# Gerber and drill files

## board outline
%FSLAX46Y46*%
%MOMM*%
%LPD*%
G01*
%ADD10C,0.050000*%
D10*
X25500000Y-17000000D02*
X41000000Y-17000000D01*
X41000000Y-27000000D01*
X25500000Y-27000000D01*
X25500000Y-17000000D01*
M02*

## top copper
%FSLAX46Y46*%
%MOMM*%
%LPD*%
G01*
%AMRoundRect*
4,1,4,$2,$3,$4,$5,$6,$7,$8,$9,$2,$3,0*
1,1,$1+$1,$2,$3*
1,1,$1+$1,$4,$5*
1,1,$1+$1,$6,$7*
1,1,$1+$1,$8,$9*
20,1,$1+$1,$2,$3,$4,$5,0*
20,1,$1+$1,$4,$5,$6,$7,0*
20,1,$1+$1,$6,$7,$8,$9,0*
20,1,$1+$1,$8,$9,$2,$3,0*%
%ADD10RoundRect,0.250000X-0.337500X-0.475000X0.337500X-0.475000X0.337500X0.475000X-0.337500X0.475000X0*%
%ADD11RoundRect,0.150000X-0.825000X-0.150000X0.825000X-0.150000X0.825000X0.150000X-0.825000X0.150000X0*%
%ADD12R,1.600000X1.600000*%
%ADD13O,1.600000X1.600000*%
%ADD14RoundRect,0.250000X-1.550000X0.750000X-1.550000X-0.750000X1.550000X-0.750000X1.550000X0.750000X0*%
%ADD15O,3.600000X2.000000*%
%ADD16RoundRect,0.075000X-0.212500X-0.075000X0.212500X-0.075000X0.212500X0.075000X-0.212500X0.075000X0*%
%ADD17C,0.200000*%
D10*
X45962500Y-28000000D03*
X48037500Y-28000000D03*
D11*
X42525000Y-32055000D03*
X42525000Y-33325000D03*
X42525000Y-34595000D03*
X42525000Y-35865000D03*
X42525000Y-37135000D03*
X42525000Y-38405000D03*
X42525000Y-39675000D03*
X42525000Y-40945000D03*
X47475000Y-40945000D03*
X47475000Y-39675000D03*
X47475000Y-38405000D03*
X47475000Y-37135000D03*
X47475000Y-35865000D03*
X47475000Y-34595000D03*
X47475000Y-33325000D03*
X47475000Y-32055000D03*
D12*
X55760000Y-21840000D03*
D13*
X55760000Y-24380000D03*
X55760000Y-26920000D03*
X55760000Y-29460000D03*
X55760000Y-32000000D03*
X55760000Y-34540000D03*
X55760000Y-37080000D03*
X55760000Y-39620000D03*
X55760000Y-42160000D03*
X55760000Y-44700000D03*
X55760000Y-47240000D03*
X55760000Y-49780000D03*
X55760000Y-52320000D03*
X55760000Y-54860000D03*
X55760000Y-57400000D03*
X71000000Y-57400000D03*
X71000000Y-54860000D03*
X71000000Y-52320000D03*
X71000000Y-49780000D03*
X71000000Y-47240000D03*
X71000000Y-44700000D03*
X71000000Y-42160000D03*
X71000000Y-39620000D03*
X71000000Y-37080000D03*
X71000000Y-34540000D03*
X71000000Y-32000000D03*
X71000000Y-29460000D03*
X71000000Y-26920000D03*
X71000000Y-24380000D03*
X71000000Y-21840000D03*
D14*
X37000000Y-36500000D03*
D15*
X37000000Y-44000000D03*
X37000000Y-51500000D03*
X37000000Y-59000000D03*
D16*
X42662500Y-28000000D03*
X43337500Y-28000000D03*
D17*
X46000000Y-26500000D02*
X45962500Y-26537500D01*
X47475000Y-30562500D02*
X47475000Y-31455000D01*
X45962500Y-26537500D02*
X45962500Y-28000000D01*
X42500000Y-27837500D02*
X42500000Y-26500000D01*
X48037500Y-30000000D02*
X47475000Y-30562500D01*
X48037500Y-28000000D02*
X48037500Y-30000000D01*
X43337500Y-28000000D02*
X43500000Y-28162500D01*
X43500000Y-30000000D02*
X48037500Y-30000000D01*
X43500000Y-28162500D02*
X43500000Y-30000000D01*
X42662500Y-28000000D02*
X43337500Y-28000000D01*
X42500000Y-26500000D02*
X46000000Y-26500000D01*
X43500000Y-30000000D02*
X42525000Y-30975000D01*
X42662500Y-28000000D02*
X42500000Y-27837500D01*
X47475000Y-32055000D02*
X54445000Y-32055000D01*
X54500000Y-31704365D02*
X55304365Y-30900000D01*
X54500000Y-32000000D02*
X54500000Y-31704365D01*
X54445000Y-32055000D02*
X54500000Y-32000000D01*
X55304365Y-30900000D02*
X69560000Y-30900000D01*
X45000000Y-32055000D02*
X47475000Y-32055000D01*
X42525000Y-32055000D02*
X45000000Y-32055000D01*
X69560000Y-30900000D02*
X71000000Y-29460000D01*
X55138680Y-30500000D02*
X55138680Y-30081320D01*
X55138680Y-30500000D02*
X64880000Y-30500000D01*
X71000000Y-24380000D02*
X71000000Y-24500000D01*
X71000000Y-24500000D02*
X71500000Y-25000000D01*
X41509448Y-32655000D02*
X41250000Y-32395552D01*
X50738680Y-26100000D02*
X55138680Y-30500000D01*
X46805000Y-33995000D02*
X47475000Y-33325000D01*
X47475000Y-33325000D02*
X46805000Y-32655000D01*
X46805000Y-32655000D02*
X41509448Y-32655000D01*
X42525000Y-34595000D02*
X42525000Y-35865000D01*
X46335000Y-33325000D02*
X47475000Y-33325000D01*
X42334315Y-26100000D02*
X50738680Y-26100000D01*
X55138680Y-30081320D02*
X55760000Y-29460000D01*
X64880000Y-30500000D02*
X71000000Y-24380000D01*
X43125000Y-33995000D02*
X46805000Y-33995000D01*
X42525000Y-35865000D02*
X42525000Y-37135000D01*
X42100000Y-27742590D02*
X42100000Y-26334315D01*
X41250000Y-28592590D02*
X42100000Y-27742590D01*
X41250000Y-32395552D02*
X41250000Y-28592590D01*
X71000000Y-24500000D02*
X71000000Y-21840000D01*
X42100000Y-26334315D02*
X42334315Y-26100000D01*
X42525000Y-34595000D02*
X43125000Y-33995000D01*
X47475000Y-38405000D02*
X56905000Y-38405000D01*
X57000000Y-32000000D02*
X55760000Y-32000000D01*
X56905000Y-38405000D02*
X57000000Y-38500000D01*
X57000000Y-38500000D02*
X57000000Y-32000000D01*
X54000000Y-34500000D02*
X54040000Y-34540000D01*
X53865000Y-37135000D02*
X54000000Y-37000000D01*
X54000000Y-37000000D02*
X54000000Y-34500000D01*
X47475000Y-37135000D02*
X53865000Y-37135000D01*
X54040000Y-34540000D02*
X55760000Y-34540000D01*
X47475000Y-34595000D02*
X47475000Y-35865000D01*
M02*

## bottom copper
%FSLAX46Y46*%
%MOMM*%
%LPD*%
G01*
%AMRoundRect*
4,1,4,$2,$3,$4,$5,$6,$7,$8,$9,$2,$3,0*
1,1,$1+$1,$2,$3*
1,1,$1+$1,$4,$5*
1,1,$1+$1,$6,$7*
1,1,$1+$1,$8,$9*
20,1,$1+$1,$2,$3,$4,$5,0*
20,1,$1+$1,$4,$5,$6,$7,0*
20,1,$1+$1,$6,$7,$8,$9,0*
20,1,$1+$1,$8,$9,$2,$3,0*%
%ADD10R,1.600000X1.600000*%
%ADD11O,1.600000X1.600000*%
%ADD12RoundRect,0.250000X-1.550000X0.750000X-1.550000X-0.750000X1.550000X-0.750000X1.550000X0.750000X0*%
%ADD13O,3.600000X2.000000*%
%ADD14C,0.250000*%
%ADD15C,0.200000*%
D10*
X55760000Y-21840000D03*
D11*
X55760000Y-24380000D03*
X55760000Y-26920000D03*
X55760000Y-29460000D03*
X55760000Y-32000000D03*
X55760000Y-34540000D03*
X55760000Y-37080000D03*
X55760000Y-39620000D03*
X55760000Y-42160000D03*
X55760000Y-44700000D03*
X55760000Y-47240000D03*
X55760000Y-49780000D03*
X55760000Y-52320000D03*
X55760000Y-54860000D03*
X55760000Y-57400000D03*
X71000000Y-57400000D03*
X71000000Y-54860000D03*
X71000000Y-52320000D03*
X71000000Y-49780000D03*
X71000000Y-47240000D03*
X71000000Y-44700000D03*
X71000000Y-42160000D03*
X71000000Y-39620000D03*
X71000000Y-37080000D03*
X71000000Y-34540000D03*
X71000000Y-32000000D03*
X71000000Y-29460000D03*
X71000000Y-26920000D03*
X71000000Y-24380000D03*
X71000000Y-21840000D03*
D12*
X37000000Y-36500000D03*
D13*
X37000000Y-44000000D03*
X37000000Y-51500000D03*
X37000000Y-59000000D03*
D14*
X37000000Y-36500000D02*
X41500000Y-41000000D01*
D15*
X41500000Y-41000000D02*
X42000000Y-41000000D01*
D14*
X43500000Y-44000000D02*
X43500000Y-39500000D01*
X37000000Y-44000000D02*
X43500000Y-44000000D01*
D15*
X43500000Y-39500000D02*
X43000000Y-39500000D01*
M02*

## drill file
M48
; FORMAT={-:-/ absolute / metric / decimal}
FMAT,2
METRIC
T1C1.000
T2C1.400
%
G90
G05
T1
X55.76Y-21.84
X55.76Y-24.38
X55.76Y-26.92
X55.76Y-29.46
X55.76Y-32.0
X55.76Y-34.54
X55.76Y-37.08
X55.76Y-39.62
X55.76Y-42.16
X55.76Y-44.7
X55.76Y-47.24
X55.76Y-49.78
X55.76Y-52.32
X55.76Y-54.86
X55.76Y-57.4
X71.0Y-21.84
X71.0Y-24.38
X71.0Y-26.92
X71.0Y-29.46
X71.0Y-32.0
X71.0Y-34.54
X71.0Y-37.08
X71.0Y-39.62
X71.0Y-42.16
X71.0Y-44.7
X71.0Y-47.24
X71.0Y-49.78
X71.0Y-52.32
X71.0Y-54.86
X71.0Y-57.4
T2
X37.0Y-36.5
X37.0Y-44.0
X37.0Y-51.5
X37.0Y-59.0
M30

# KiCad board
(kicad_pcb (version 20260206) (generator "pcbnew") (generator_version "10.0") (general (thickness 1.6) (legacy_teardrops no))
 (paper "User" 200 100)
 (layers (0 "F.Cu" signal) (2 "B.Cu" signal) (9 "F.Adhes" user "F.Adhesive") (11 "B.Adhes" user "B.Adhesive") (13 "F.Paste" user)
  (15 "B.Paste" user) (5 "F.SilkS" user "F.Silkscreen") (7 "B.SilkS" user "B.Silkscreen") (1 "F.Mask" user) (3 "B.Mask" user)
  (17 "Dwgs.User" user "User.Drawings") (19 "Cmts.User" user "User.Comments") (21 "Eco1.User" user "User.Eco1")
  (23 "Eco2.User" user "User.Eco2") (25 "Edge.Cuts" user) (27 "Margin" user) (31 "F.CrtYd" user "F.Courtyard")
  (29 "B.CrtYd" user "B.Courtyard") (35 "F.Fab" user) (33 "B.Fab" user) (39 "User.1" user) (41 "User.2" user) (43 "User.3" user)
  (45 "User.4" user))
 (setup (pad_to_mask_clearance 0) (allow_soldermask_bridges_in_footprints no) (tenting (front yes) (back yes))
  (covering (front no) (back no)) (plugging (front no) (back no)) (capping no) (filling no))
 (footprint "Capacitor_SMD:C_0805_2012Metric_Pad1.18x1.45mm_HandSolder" (layer "F.Cu") (at 47 28)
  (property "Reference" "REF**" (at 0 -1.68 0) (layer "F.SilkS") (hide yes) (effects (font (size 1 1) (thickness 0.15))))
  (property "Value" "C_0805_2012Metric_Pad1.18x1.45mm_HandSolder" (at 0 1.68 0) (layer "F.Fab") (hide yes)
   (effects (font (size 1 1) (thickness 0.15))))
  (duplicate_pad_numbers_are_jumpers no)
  (pad "1" smd roundrect (at -1.0375 0) (size 1.175 1.45) (layers "F.Cu" "F.Mask" "F.Paste") (roundrect_rratio 0.212766))
  (pad "2" smd roundrect (at 1.0375 0) (size 1.175 1.45) (layers "F.Cu" "F.Mask" "F.Paste") (roundrect_rratio 0.212766)))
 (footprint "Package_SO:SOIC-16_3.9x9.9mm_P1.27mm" (layer "F.Cu") (at 45 36.5)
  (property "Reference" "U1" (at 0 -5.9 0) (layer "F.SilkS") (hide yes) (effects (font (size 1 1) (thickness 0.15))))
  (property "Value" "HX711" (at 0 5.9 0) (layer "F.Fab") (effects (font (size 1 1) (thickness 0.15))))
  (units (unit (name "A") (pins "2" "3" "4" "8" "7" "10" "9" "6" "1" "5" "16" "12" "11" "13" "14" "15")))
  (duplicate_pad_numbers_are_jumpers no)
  (pad "1" smd roundrect (at -2.475 -4.445) (size 1.95 0.6) (layers "F.Cu" "F.Mask" "F.Paste") (roundrect_rratio 0.25)
   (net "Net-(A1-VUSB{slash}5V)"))
  (pad "2" smd roundrect (at -2.475 -3.175) (size 1.95 0.6) (layers "F.Cu" "F.Mask" "F.Paste") (roundrect_rratio 0.25)
   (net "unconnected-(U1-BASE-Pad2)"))
  (pad "3" smd roundrect (at -2.475 -1.905) (size 1.95 0.6) (layers "F.Cu" "F.Mask" "F.Paste") (roundrect_rratio 0.25) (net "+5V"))
  (pad "4" smd roundrect (at -2.475 -0.635) (size 1.95 0.6) (layers "F.Cu" "F.Mask" "F.Paste") (roundrect_rratio 0.25) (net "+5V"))
  (pad "5" smd roundrect (at -2.475 0.635) (size 1.95 0.6) (layers "F.Cu" "F.Mask" "F.Paste") (roundrect_rratio 0.25) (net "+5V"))
  (pad "6" smd roundrect (at -2.475 1.905) (size 1.95 0.6) (layers "F.Cu" "F.Mask" "F.Paste") (roundrect_rratio 0.25)
   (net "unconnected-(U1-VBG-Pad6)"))
  (pad "7" smd roundrect (at -2.475 3.175) (size 1.95 0.6) (layers "F.Cu" "F.Mask" "F.Paste") (roundrect_rratio 0.25) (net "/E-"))
  (pad "8" smd roundrect (at -2.475 4.445) (size 1.95 0.6) (layers "F.Cu" "F.Mask" "F.Paste") (roundrect_rratio 0.25) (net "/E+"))
  (pad "9" smd roundrect (at 2.475 4.445) (size 1.95 0.6) (layers "F.Cu" "F.Mask" "F.Paste") (roundrect_rratio 0.25)
   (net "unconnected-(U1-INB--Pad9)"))
  (pad "10" smd roundrect (at 2.475 3.175) (size 1.95 0.6) (layers "F.Cu" "F.Mask" "F.Paste") (roundrect_rratio 0.25)
   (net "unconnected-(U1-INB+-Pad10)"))
  (pad "11" smd roundrect (at 2.475 1.905) (size 1.95 0.6) (layers "F.Cu" "F.Mask" "F.Paste") (roundrect_rratio 0.25) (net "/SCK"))
  (pad "12" smd roundrect (at 2.475 0.635) (size 1.95 0.6) (layers "F.Cu" "F.Mask" "F.Paste") (roundrect_rratio 0.25) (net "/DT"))
  (pad "13" smd roundrect (at 2.475 -0.635) (size 1.95 0.6) (layers "F.Cu" "F.Mask" "F.Paste") (roundrect_rratio 0.25) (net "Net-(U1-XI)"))
  (pad "14" smd roundrect (at 2.475 -1.905) (size 1.95 0.6) (layers "F.Cu" "F.Mask" "F.Paste") (roundrect_rratio 0.25) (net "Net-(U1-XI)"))
  (pad "15" smd roundrect (at 2.475 -3.175) (size 1.95 0.6) (layers "F.Cu" "F.Mask" "F.Paste") (roundrect_rratio 0.25) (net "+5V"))
  (pad "16" smd roundrect (at 2.475 -4.445) (size 1.95 0.6) (layers "F.Cu" "F.Mask" "F.Paste") (roundrect_rratio 0.25)
   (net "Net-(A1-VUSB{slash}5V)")))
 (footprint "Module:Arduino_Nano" (layer "F.Cu") (at 55.76 21.84)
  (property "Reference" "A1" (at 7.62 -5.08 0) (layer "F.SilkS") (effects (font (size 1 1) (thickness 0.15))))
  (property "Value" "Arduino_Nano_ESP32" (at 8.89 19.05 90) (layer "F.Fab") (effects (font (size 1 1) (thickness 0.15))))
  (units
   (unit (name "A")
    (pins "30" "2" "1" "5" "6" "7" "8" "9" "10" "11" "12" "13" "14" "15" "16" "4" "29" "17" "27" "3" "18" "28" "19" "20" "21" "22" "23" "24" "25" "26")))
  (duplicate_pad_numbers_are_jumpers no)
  (pad "1" thru_hole rect (at 0 0) (size 1.6 1.6) (drill 1) (layers "*.Cu" "*.Mask") (remove_unused_layers no)
   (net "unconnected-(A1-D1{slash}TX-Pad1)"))
  (pad "2" thru_hole oval (at 0 2.54) (size 1.6 1.6) (drill 1) (layers "*.Cu" "*.Mask") (remove_unused_layers no)
   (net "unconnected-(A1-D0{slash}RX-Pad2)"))
  (pad "3" thru_hole oval (at 0 5.08) (size 1.6 1.6) (drill 1) (layers "*.Cu" "*.Mask") (remove_unused_layers no)
   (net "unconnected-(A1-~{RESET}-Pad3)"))
  (pad "4" thru_hole oval (at 0 7.62) (size 1.6 1.6) (drill 1) (layers "*.Cu" "*.Mask") (remove_unused_layers no) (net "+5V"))
  (pad "5" thru_hole oval (at 0 10.16) (size 1.6 1.6) (drill 1) (layers "*.Cu" "*.Mask") (remove_unused_layers no) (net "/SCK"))
  (pad "6" thru_hole oval (at 0 12.7) (size 1.6 1.6) (drill 1) (layers "*.Cu" "*.Mask") (remove_unused_layers no) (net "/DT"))
  (pad "7" thru_hole oval (at 0 15.24) (size 1.6 1.6) (drill 1) (layers "*.Cu" "*.Mask") (remove_unused_layers no)
   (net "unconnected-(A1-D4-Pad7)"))
  (pad "8" thru_hole oval (at 0 17.78) (size 1.6 1.6) (drill 1) (layers "*.Cu" "*.Mask") (remove_unused_layers no)
   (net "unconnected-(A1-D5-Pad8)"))
  (pad "9" thru_hole oval (at 0 20.32) (size 1.6 1.6) (drill 1) (layers "*.Cu" "*.Mask") (remove_unused_layers no)
   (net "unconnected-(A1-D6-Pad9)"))
  (pad "10" thru_hole oval (at 0 22.86) (size 1.6 1.6) (drill 1) (layers "*.Cu" "*.Mask") (remove_unused_layers no)
   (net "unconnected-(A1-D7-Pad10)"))
  (pad "11" thru_hole oval (at 0 25.4) (size 1.6 1.6) (drill 1) (layers "*.Cu" "*.Mask") (remove_unused_layers no)
   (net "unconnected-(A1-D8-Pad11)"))
  (pad "12" thru_hole oval (at 0 27.94) (size 1.6 1.6) (drill 1) (layers "*.Cu" "*.Mask") (remove_unused_layers no)
   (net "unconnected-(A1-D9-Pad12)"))
  (pad "13" thru_hole oval (at 0 30.48) (size 1.6 1.6) (drill 1) (layers "*.Cu" "*.Mask") (remove_unused_layers no)
   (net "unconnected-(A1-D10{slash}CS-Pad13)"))
  (pad "14" thru_hole oval (at 0 33.02) (size 1.6 1.6) (drill 1) (layers "*.Cu" "*.Mask") (remove_unused_layers no)
   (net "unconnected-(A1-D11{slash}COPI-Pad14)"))
  (pad "15" thru_hole oval (at 0 35.56) (size 1.6 1.6) (drill 1) (layers "*.Cu" "*.Mask") (remove_unused_layers no)
   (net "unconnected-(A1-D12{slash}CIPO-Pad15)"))
  (pad "16" thru_hole oval (at 15.24 35.56) (size 1.6 1.6) (drill 1) (layers "*.Cu" "*.Mask") (remove_unused_layers no)
   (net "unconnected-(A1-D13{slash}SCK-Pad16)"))
  (pad "17" thru_hole oval (at 15.24 33.02) (size 1.6 1.6) (drill 1) (layers "*.Cu" "*.Mask") (remove_unused_layers no)
   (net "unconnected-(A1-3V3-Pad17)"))
  (pad "18" thru_hole oval (at 15.24 30.48) (size 1.6 1.6) (drill 1) (layers "*.Cu" "*.Mask") (remove_unused_layers no)
   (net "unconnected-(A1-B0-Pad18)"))
  (pad "19" thru_hole oval (at 15.24 27.94) (size 1.6 1.6) (drill 1) (layers "*.Cu" "*.Mask") (remove_unused_layers no)
   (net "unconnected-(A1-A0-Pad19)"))
  (pad "20" thru_hole oval (at 15.24 25.4) (size 1.6 1.6) (drill 1) (layers "*.Cu" "*.Mask") (remove_unused_layers no)
   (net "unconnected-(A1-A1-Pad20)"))
  (pad "21" thru_hole oval (at 15.24 22.86) (size 1.6 1.6) (drill 1) (layers "*.Cu" "*.Mask") (remove_unused_layers no)
   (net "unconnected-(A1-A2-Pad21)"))
  (pad "22" thru_hole oval (at 15.24 20.32) (size 1.6 1.6) (drill 1) (layers "*.Cu" "*.Mask") (remove_unused_layers no)
   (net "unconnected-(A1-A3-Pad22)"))
  (pad "23" thru_hole oval (at 15.24 17.78) (size 1.6 1.6) (drill 1) (layers "*.Cu" "*.Mask") (remove_unused_layers no)
   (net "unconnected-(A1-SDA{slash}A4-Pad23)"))
  (pad "24" thru_hole oval (at 15.24 15.24) (size 1.6 1.6) (drill 1) (layers "*.Cu" "*.Mask") (remove_unused_layers no)
   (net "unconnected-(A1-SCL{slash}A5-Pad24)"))
  (pad "25" thru_hole oval (at 15.24 12.7) (size 1.6 1.6) (drill 1) (layers "*.Cu" "*.Mask") (remove_unused_layers no)
   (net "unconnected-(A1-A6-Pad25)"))
  (pad "26" thru_hole oval (at 15.24 10.16) (size 1.6 1.6) (drill 1) (layers "*.Cu" "*.Mask") (remove_unused_layers no)
   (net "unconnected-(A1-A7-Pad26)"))
  (pad "27" thru_hole oval (at 15.24 7.62) (size 1.6 1.6) (drill 1) (layers "*.Cu" "*.Mask") (remove_unused_layers no)
   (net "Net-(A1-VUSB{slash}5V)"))
  (pad "28" thru_hole oval (at 15.24 5.08) (size 1.6 1.6) (drill 1) (layers "*.Cu" "*.Mask") (remove_unused_layers no)
   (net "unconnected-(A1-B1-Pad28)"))
  (pad "29" thru_hole oval (at 15.24 2.54) (size 1.6 1.6) (drill 1) (layers "*.Cu" "*.Mask") (remove_unused_layers no) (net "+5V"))
  (pad "30" thru_hole oval (at 15.24 0) (size 1.6 1.6) (drill 1) (layers "*.Cu" "*.Mask") (remove_unused_layers no) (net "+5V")))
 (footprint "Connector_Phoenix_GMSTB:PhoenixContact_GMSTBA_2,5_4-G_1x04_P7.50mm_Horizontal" (layer "F.Cu") (at 37 36.5 -90)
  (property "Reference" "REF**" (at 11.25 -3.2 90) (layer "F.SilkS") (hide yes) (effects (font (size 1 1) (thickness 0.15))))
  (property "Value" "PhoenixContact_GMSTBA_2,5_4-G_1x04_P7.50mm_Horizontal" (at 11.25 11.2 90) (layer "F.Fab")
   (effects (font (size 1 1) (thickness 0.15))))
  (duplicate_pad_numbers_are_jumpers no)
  (pad "1" thru_hole roundrect (at 0 0 270) (size 2 3.6) (drill 1.4) (layers "*.Cu" "*.Mask") (remove_unused_layers no)
   (roundrect_rratio 0.125))
  (pad "2" thru_hole oval (at 7.5 0 270) (size 2 3.6) (drill 1.4) (layers "*.Cu" "*.Mask") (remove_unused_layers no))
  (pad "3" thru_hole oval (at 15 0 270) (size 2 3.6) (drill 1.4) (layers "*.Cu" "*.Mask") (remove_unused_layers no))
  (pad "4" thru_hole oval (at 22.5 0 270) (size 2 3.6) (drill 1.4) (layers "*.Cu" "*.Mask") (remove_unused_layers no)))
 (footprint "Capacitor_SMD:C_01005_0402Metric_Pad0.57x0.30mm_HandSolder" (layer "F.Cu") (at 43 28)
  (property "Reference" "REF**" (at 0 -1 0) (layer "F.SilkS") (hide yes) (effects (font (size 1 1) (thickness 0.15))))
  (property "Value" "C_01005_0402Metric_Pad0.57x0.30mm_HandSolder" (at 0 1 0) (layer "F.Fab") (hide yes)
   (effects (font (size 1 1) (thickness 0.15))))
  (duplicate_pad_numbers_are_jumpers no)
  (pad "" smd roundrect (at -0.3625 0) (size 0.41 0.27) (layers "F.Paste") (roundrect_rratio 0.25))
  (pad "" smd roundrect (at 0.3625 0) (size 0.41 0.27) (layers "F.Paste") (roundrect_rratio 0.25))
  (pad "1" smd roundrect (at -0.3375 0) (size 0.575 0.3) (layers "F.Cu" "F.Mask") (roundrect_rratio 0.25))
  (pad "2" smd roundrect (at 0.3375 0) (size 0.575 0.3) (layers "F.Cu" "F.Mask") (roundrect_rratio 0.25)))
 (gr_rect (start 25.5 17) (end 41 27) (stroke (width 0.05) (type default)) (fill no) (layer "Edge.Cuts"))
 (segment (start 46 26.5) (end 45.9625 26.5375) (width 0.2) (layer "F.Cu") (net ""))
 (segment (start 47.475 30.5625) (end 47.475 31.455) (width 0.2) (layer "F.Cu") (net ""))
 (segment (start 45.9625 26.5375) (end 45.9625 28) (width 0.2) (layer "F.Cu") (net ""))
 (segment (start 42.5 27.8375) (end 42.5 26.5) (width 0.2) (layer "F.Cu") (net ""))
 (segment (start 48.0375 30) (end 47.475 30.5625) (width 0.2) (layer "F.Cu") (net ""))
 (segment (start 48.0375 28) (end 48.0375 30) (width 0.2) (layer "F.Cu") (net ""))
 (segment (start 43.3375 28) (end 43.5 28.1625) (width 0.2) (layer "F.Cu") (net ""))
 (segment (start 43.5 30) (end 48.0375 30) (width 0.2) (layer "F.Cu") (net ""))
 (segment (start 43.5 28.1625) (end 43.5 30) (width 0.2) (layer "F.Cu") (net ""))
 (segment (start 42.6625 28) (end 43.3375 28) (width 0.2) (layer "F.Cu") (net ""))
 (segment (start 42.5 26.5) (end 46 26.5) (width 0.2) (layer "F.Cu") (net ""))
 (segment (start 43.5 30) (end 42.525 30.975) (width 0.2) (layer "F.Cu") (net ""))
 (segment (start 42.6625 28) (end 42.5 27.8375) (width 0.2) (layer "F.Cu") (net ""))
 (segment (start 37 36.5) (end 41.5 41) (width 0.25) (layer "B.Cu") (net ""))
 (segment (start 41.5 41) (end 42 41) (width 0.2) (layer "B.Cu") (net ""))
 (segment (start 43.5 44) (end 43.5 39.5) (width 0.25) (layer "B.Cu") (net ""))
 (segment (start 37 44) (end 43.5 44) (width 0.25) (layer "B.Cu") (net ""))
 (segment (start 43.5 39.5) (end 43 39.5) (width 0.2) (layer "B.Cu") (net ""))
 (segment (start 47.475 32.055) (end 54.445 32.055) (width 0.2) (layer "F.Cu") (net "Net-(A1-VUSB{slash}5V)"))
 (segment (start 54.5 31.704365) (end 55.304365 30.9) (width 0.2) (layer "F.Cu") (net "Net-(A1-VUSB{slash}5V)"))
 (segment (start 54.5 32) (end 54.5 31.704365) (width 0.2) (layer "F.Cu") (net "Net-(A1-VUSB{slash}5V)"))
 (segment (start 54.445 32.055) (end 54.5 32) (width 0.2) (layer "F.Cu") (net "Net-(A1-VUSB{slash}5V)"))
 (segment (start 55.304365 30.9) (end 69.56 30.9) (width 0.2) (layer "F.Cu") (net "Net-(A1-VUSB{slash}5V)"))
 (segment (start 45 32.055) (end 47.475 32.055) (width 0.2) (layer "F.Cu") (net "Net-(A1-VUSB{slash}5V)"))
 (segment (start 42.525 32.055) (end 45 32.055) (width 0.2) (layer "F.Cu") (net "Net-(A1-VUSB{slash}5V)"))
 (segment (start 69.56 30.9) (end 71 29.46) (width 0.2) (layer "F.Cu") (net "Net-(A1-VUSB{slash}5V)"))
 (segment (start 55.13868 30.5) (end 55.13868 30.08132) (width 0.2) (layer "F.Cu") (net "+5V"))
 (segment (start 55.13868 30.5) (end 64.88 30.5) (width 0.2) (layer "F.Cu") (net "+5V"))
 (segment (start 71 24.38) (end 71 24.5) (width 0.2) (layer "F.Cu") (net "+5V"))
 (segment (start 71 24.5) (end 71.5 25) (width 0.2) (layer "F.Cu") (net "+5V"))
 (segment (start 41.509448 32.655) (end 41.25 32.395552) (width 0.2) (layer "F.Cu") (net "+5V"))
 (segment (start 50.73868 26.1) (end 55.13868 30.5) (width 0.2) (layer "F.Cu") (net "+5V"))
 (segment (start 46.805 33.995) (end 47.475 33.325) (width 0.2) (layer "F.Cu") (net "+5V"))
 (segment (start 47.475 33.325) (end 46.805 32.655) (width 0.2) (layer "F.Cu") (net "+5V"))
 (segment (start 46.805 32.655) (end 41.509448 32.655) (width 0.2) (layer "F.Cu") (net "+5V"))
 (segment (start 42.525 34.595) (end 42.525 35.865) (width 0.2) (layer "F.Cu") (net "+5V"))
 (segment (start 46.335 33.325) (end 47.475 33.325) (width 0.2) (layer "F.Cu") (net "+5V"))
 (segment (start 42.334315 26.1) (end 50.73868 26.1) (width 0.2) (layer "F.Cu") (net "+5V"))
 (segment (start 55.13868 30.08132) (end 55.76 29.46) (width 0.2) (layer "F.Cu") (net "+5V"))
 (segment (start 64.88 30.5) (end 71 24.38) (width 0.2) (layer "F.Cu") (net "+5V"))
 (segment (start 43.125 33.995) (end 46.805 33.995) (width 0.2) (layer "F.Cu") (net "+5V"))
 (segment (start 42.525 35.865) (end 42.525 37.135) (width 0.2) (layer "F.Cu") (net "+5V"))
 (segment (start 42.1 27.74259) (end 42.1 26.334315) (width 0.2) (layer "F.Cu") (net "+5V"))
 (segment (start 41.25 28.59259) (end 42.1 27.74259) (width 0.2) (layer "F.Cu") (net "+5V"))
 (segment (start 41.25 32.395552) (end 41.25 28.59259) (width 0.2) (layer "F.Cu") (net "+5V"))
 (segment (start 71 24.5) (end 71 21.84) (width 0.2) (layer "F.Cu") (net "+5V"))
 (segment (start 42.1 26.334315) (end 42.334315 26.1) (width 0.2) (layer "F.Cu") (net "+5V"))
 (segment (start 42.525 34.595) (end 43.125 33.995) (width 0.2) (layer "F.Cu") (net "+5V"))
 (segment (start 47.475 38.405) (end 56.905 38.405) (width 0.2) (layer "F.Cu") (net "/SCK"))
 (segment (start 57 32) (end 55.76 32) (width 0.2) (layer "F.Cu") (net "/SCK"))
 (segment (start 56.905 38.405) (end 57 38.5) (width 0.2) (layer "F.Cu") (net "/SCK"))
 (segment (start 57 38.5) (end 57 32) (width 0.2) (layer "F.Cu") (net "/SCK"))
 (segment (start 54 34.5) (end 54.04 34.54) (width 0.2) (layer "F.Cu") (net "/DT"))
 (segment (start 53.865 37.135) (end 54 37) (width 0.2) (layer "F.Cu") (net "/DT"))
 (segment (start 54 37) (end 54 34.5) (width 0.2) (layer "F.Cu") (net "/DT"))
 (segment (start 47.475 37.135) (end 53.865 37.135) (width 0.2) (layer "F.Cu") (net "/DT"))
 (segment (start 54.04 34.54) (end 55.76 34.54) (width 0.2) (layer "F.Cu") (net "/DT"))
 (segment (start 47.475 34.595) (end 47.475 35.865) (width 0.2) (layer "F.Cu") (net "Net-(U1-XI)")))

